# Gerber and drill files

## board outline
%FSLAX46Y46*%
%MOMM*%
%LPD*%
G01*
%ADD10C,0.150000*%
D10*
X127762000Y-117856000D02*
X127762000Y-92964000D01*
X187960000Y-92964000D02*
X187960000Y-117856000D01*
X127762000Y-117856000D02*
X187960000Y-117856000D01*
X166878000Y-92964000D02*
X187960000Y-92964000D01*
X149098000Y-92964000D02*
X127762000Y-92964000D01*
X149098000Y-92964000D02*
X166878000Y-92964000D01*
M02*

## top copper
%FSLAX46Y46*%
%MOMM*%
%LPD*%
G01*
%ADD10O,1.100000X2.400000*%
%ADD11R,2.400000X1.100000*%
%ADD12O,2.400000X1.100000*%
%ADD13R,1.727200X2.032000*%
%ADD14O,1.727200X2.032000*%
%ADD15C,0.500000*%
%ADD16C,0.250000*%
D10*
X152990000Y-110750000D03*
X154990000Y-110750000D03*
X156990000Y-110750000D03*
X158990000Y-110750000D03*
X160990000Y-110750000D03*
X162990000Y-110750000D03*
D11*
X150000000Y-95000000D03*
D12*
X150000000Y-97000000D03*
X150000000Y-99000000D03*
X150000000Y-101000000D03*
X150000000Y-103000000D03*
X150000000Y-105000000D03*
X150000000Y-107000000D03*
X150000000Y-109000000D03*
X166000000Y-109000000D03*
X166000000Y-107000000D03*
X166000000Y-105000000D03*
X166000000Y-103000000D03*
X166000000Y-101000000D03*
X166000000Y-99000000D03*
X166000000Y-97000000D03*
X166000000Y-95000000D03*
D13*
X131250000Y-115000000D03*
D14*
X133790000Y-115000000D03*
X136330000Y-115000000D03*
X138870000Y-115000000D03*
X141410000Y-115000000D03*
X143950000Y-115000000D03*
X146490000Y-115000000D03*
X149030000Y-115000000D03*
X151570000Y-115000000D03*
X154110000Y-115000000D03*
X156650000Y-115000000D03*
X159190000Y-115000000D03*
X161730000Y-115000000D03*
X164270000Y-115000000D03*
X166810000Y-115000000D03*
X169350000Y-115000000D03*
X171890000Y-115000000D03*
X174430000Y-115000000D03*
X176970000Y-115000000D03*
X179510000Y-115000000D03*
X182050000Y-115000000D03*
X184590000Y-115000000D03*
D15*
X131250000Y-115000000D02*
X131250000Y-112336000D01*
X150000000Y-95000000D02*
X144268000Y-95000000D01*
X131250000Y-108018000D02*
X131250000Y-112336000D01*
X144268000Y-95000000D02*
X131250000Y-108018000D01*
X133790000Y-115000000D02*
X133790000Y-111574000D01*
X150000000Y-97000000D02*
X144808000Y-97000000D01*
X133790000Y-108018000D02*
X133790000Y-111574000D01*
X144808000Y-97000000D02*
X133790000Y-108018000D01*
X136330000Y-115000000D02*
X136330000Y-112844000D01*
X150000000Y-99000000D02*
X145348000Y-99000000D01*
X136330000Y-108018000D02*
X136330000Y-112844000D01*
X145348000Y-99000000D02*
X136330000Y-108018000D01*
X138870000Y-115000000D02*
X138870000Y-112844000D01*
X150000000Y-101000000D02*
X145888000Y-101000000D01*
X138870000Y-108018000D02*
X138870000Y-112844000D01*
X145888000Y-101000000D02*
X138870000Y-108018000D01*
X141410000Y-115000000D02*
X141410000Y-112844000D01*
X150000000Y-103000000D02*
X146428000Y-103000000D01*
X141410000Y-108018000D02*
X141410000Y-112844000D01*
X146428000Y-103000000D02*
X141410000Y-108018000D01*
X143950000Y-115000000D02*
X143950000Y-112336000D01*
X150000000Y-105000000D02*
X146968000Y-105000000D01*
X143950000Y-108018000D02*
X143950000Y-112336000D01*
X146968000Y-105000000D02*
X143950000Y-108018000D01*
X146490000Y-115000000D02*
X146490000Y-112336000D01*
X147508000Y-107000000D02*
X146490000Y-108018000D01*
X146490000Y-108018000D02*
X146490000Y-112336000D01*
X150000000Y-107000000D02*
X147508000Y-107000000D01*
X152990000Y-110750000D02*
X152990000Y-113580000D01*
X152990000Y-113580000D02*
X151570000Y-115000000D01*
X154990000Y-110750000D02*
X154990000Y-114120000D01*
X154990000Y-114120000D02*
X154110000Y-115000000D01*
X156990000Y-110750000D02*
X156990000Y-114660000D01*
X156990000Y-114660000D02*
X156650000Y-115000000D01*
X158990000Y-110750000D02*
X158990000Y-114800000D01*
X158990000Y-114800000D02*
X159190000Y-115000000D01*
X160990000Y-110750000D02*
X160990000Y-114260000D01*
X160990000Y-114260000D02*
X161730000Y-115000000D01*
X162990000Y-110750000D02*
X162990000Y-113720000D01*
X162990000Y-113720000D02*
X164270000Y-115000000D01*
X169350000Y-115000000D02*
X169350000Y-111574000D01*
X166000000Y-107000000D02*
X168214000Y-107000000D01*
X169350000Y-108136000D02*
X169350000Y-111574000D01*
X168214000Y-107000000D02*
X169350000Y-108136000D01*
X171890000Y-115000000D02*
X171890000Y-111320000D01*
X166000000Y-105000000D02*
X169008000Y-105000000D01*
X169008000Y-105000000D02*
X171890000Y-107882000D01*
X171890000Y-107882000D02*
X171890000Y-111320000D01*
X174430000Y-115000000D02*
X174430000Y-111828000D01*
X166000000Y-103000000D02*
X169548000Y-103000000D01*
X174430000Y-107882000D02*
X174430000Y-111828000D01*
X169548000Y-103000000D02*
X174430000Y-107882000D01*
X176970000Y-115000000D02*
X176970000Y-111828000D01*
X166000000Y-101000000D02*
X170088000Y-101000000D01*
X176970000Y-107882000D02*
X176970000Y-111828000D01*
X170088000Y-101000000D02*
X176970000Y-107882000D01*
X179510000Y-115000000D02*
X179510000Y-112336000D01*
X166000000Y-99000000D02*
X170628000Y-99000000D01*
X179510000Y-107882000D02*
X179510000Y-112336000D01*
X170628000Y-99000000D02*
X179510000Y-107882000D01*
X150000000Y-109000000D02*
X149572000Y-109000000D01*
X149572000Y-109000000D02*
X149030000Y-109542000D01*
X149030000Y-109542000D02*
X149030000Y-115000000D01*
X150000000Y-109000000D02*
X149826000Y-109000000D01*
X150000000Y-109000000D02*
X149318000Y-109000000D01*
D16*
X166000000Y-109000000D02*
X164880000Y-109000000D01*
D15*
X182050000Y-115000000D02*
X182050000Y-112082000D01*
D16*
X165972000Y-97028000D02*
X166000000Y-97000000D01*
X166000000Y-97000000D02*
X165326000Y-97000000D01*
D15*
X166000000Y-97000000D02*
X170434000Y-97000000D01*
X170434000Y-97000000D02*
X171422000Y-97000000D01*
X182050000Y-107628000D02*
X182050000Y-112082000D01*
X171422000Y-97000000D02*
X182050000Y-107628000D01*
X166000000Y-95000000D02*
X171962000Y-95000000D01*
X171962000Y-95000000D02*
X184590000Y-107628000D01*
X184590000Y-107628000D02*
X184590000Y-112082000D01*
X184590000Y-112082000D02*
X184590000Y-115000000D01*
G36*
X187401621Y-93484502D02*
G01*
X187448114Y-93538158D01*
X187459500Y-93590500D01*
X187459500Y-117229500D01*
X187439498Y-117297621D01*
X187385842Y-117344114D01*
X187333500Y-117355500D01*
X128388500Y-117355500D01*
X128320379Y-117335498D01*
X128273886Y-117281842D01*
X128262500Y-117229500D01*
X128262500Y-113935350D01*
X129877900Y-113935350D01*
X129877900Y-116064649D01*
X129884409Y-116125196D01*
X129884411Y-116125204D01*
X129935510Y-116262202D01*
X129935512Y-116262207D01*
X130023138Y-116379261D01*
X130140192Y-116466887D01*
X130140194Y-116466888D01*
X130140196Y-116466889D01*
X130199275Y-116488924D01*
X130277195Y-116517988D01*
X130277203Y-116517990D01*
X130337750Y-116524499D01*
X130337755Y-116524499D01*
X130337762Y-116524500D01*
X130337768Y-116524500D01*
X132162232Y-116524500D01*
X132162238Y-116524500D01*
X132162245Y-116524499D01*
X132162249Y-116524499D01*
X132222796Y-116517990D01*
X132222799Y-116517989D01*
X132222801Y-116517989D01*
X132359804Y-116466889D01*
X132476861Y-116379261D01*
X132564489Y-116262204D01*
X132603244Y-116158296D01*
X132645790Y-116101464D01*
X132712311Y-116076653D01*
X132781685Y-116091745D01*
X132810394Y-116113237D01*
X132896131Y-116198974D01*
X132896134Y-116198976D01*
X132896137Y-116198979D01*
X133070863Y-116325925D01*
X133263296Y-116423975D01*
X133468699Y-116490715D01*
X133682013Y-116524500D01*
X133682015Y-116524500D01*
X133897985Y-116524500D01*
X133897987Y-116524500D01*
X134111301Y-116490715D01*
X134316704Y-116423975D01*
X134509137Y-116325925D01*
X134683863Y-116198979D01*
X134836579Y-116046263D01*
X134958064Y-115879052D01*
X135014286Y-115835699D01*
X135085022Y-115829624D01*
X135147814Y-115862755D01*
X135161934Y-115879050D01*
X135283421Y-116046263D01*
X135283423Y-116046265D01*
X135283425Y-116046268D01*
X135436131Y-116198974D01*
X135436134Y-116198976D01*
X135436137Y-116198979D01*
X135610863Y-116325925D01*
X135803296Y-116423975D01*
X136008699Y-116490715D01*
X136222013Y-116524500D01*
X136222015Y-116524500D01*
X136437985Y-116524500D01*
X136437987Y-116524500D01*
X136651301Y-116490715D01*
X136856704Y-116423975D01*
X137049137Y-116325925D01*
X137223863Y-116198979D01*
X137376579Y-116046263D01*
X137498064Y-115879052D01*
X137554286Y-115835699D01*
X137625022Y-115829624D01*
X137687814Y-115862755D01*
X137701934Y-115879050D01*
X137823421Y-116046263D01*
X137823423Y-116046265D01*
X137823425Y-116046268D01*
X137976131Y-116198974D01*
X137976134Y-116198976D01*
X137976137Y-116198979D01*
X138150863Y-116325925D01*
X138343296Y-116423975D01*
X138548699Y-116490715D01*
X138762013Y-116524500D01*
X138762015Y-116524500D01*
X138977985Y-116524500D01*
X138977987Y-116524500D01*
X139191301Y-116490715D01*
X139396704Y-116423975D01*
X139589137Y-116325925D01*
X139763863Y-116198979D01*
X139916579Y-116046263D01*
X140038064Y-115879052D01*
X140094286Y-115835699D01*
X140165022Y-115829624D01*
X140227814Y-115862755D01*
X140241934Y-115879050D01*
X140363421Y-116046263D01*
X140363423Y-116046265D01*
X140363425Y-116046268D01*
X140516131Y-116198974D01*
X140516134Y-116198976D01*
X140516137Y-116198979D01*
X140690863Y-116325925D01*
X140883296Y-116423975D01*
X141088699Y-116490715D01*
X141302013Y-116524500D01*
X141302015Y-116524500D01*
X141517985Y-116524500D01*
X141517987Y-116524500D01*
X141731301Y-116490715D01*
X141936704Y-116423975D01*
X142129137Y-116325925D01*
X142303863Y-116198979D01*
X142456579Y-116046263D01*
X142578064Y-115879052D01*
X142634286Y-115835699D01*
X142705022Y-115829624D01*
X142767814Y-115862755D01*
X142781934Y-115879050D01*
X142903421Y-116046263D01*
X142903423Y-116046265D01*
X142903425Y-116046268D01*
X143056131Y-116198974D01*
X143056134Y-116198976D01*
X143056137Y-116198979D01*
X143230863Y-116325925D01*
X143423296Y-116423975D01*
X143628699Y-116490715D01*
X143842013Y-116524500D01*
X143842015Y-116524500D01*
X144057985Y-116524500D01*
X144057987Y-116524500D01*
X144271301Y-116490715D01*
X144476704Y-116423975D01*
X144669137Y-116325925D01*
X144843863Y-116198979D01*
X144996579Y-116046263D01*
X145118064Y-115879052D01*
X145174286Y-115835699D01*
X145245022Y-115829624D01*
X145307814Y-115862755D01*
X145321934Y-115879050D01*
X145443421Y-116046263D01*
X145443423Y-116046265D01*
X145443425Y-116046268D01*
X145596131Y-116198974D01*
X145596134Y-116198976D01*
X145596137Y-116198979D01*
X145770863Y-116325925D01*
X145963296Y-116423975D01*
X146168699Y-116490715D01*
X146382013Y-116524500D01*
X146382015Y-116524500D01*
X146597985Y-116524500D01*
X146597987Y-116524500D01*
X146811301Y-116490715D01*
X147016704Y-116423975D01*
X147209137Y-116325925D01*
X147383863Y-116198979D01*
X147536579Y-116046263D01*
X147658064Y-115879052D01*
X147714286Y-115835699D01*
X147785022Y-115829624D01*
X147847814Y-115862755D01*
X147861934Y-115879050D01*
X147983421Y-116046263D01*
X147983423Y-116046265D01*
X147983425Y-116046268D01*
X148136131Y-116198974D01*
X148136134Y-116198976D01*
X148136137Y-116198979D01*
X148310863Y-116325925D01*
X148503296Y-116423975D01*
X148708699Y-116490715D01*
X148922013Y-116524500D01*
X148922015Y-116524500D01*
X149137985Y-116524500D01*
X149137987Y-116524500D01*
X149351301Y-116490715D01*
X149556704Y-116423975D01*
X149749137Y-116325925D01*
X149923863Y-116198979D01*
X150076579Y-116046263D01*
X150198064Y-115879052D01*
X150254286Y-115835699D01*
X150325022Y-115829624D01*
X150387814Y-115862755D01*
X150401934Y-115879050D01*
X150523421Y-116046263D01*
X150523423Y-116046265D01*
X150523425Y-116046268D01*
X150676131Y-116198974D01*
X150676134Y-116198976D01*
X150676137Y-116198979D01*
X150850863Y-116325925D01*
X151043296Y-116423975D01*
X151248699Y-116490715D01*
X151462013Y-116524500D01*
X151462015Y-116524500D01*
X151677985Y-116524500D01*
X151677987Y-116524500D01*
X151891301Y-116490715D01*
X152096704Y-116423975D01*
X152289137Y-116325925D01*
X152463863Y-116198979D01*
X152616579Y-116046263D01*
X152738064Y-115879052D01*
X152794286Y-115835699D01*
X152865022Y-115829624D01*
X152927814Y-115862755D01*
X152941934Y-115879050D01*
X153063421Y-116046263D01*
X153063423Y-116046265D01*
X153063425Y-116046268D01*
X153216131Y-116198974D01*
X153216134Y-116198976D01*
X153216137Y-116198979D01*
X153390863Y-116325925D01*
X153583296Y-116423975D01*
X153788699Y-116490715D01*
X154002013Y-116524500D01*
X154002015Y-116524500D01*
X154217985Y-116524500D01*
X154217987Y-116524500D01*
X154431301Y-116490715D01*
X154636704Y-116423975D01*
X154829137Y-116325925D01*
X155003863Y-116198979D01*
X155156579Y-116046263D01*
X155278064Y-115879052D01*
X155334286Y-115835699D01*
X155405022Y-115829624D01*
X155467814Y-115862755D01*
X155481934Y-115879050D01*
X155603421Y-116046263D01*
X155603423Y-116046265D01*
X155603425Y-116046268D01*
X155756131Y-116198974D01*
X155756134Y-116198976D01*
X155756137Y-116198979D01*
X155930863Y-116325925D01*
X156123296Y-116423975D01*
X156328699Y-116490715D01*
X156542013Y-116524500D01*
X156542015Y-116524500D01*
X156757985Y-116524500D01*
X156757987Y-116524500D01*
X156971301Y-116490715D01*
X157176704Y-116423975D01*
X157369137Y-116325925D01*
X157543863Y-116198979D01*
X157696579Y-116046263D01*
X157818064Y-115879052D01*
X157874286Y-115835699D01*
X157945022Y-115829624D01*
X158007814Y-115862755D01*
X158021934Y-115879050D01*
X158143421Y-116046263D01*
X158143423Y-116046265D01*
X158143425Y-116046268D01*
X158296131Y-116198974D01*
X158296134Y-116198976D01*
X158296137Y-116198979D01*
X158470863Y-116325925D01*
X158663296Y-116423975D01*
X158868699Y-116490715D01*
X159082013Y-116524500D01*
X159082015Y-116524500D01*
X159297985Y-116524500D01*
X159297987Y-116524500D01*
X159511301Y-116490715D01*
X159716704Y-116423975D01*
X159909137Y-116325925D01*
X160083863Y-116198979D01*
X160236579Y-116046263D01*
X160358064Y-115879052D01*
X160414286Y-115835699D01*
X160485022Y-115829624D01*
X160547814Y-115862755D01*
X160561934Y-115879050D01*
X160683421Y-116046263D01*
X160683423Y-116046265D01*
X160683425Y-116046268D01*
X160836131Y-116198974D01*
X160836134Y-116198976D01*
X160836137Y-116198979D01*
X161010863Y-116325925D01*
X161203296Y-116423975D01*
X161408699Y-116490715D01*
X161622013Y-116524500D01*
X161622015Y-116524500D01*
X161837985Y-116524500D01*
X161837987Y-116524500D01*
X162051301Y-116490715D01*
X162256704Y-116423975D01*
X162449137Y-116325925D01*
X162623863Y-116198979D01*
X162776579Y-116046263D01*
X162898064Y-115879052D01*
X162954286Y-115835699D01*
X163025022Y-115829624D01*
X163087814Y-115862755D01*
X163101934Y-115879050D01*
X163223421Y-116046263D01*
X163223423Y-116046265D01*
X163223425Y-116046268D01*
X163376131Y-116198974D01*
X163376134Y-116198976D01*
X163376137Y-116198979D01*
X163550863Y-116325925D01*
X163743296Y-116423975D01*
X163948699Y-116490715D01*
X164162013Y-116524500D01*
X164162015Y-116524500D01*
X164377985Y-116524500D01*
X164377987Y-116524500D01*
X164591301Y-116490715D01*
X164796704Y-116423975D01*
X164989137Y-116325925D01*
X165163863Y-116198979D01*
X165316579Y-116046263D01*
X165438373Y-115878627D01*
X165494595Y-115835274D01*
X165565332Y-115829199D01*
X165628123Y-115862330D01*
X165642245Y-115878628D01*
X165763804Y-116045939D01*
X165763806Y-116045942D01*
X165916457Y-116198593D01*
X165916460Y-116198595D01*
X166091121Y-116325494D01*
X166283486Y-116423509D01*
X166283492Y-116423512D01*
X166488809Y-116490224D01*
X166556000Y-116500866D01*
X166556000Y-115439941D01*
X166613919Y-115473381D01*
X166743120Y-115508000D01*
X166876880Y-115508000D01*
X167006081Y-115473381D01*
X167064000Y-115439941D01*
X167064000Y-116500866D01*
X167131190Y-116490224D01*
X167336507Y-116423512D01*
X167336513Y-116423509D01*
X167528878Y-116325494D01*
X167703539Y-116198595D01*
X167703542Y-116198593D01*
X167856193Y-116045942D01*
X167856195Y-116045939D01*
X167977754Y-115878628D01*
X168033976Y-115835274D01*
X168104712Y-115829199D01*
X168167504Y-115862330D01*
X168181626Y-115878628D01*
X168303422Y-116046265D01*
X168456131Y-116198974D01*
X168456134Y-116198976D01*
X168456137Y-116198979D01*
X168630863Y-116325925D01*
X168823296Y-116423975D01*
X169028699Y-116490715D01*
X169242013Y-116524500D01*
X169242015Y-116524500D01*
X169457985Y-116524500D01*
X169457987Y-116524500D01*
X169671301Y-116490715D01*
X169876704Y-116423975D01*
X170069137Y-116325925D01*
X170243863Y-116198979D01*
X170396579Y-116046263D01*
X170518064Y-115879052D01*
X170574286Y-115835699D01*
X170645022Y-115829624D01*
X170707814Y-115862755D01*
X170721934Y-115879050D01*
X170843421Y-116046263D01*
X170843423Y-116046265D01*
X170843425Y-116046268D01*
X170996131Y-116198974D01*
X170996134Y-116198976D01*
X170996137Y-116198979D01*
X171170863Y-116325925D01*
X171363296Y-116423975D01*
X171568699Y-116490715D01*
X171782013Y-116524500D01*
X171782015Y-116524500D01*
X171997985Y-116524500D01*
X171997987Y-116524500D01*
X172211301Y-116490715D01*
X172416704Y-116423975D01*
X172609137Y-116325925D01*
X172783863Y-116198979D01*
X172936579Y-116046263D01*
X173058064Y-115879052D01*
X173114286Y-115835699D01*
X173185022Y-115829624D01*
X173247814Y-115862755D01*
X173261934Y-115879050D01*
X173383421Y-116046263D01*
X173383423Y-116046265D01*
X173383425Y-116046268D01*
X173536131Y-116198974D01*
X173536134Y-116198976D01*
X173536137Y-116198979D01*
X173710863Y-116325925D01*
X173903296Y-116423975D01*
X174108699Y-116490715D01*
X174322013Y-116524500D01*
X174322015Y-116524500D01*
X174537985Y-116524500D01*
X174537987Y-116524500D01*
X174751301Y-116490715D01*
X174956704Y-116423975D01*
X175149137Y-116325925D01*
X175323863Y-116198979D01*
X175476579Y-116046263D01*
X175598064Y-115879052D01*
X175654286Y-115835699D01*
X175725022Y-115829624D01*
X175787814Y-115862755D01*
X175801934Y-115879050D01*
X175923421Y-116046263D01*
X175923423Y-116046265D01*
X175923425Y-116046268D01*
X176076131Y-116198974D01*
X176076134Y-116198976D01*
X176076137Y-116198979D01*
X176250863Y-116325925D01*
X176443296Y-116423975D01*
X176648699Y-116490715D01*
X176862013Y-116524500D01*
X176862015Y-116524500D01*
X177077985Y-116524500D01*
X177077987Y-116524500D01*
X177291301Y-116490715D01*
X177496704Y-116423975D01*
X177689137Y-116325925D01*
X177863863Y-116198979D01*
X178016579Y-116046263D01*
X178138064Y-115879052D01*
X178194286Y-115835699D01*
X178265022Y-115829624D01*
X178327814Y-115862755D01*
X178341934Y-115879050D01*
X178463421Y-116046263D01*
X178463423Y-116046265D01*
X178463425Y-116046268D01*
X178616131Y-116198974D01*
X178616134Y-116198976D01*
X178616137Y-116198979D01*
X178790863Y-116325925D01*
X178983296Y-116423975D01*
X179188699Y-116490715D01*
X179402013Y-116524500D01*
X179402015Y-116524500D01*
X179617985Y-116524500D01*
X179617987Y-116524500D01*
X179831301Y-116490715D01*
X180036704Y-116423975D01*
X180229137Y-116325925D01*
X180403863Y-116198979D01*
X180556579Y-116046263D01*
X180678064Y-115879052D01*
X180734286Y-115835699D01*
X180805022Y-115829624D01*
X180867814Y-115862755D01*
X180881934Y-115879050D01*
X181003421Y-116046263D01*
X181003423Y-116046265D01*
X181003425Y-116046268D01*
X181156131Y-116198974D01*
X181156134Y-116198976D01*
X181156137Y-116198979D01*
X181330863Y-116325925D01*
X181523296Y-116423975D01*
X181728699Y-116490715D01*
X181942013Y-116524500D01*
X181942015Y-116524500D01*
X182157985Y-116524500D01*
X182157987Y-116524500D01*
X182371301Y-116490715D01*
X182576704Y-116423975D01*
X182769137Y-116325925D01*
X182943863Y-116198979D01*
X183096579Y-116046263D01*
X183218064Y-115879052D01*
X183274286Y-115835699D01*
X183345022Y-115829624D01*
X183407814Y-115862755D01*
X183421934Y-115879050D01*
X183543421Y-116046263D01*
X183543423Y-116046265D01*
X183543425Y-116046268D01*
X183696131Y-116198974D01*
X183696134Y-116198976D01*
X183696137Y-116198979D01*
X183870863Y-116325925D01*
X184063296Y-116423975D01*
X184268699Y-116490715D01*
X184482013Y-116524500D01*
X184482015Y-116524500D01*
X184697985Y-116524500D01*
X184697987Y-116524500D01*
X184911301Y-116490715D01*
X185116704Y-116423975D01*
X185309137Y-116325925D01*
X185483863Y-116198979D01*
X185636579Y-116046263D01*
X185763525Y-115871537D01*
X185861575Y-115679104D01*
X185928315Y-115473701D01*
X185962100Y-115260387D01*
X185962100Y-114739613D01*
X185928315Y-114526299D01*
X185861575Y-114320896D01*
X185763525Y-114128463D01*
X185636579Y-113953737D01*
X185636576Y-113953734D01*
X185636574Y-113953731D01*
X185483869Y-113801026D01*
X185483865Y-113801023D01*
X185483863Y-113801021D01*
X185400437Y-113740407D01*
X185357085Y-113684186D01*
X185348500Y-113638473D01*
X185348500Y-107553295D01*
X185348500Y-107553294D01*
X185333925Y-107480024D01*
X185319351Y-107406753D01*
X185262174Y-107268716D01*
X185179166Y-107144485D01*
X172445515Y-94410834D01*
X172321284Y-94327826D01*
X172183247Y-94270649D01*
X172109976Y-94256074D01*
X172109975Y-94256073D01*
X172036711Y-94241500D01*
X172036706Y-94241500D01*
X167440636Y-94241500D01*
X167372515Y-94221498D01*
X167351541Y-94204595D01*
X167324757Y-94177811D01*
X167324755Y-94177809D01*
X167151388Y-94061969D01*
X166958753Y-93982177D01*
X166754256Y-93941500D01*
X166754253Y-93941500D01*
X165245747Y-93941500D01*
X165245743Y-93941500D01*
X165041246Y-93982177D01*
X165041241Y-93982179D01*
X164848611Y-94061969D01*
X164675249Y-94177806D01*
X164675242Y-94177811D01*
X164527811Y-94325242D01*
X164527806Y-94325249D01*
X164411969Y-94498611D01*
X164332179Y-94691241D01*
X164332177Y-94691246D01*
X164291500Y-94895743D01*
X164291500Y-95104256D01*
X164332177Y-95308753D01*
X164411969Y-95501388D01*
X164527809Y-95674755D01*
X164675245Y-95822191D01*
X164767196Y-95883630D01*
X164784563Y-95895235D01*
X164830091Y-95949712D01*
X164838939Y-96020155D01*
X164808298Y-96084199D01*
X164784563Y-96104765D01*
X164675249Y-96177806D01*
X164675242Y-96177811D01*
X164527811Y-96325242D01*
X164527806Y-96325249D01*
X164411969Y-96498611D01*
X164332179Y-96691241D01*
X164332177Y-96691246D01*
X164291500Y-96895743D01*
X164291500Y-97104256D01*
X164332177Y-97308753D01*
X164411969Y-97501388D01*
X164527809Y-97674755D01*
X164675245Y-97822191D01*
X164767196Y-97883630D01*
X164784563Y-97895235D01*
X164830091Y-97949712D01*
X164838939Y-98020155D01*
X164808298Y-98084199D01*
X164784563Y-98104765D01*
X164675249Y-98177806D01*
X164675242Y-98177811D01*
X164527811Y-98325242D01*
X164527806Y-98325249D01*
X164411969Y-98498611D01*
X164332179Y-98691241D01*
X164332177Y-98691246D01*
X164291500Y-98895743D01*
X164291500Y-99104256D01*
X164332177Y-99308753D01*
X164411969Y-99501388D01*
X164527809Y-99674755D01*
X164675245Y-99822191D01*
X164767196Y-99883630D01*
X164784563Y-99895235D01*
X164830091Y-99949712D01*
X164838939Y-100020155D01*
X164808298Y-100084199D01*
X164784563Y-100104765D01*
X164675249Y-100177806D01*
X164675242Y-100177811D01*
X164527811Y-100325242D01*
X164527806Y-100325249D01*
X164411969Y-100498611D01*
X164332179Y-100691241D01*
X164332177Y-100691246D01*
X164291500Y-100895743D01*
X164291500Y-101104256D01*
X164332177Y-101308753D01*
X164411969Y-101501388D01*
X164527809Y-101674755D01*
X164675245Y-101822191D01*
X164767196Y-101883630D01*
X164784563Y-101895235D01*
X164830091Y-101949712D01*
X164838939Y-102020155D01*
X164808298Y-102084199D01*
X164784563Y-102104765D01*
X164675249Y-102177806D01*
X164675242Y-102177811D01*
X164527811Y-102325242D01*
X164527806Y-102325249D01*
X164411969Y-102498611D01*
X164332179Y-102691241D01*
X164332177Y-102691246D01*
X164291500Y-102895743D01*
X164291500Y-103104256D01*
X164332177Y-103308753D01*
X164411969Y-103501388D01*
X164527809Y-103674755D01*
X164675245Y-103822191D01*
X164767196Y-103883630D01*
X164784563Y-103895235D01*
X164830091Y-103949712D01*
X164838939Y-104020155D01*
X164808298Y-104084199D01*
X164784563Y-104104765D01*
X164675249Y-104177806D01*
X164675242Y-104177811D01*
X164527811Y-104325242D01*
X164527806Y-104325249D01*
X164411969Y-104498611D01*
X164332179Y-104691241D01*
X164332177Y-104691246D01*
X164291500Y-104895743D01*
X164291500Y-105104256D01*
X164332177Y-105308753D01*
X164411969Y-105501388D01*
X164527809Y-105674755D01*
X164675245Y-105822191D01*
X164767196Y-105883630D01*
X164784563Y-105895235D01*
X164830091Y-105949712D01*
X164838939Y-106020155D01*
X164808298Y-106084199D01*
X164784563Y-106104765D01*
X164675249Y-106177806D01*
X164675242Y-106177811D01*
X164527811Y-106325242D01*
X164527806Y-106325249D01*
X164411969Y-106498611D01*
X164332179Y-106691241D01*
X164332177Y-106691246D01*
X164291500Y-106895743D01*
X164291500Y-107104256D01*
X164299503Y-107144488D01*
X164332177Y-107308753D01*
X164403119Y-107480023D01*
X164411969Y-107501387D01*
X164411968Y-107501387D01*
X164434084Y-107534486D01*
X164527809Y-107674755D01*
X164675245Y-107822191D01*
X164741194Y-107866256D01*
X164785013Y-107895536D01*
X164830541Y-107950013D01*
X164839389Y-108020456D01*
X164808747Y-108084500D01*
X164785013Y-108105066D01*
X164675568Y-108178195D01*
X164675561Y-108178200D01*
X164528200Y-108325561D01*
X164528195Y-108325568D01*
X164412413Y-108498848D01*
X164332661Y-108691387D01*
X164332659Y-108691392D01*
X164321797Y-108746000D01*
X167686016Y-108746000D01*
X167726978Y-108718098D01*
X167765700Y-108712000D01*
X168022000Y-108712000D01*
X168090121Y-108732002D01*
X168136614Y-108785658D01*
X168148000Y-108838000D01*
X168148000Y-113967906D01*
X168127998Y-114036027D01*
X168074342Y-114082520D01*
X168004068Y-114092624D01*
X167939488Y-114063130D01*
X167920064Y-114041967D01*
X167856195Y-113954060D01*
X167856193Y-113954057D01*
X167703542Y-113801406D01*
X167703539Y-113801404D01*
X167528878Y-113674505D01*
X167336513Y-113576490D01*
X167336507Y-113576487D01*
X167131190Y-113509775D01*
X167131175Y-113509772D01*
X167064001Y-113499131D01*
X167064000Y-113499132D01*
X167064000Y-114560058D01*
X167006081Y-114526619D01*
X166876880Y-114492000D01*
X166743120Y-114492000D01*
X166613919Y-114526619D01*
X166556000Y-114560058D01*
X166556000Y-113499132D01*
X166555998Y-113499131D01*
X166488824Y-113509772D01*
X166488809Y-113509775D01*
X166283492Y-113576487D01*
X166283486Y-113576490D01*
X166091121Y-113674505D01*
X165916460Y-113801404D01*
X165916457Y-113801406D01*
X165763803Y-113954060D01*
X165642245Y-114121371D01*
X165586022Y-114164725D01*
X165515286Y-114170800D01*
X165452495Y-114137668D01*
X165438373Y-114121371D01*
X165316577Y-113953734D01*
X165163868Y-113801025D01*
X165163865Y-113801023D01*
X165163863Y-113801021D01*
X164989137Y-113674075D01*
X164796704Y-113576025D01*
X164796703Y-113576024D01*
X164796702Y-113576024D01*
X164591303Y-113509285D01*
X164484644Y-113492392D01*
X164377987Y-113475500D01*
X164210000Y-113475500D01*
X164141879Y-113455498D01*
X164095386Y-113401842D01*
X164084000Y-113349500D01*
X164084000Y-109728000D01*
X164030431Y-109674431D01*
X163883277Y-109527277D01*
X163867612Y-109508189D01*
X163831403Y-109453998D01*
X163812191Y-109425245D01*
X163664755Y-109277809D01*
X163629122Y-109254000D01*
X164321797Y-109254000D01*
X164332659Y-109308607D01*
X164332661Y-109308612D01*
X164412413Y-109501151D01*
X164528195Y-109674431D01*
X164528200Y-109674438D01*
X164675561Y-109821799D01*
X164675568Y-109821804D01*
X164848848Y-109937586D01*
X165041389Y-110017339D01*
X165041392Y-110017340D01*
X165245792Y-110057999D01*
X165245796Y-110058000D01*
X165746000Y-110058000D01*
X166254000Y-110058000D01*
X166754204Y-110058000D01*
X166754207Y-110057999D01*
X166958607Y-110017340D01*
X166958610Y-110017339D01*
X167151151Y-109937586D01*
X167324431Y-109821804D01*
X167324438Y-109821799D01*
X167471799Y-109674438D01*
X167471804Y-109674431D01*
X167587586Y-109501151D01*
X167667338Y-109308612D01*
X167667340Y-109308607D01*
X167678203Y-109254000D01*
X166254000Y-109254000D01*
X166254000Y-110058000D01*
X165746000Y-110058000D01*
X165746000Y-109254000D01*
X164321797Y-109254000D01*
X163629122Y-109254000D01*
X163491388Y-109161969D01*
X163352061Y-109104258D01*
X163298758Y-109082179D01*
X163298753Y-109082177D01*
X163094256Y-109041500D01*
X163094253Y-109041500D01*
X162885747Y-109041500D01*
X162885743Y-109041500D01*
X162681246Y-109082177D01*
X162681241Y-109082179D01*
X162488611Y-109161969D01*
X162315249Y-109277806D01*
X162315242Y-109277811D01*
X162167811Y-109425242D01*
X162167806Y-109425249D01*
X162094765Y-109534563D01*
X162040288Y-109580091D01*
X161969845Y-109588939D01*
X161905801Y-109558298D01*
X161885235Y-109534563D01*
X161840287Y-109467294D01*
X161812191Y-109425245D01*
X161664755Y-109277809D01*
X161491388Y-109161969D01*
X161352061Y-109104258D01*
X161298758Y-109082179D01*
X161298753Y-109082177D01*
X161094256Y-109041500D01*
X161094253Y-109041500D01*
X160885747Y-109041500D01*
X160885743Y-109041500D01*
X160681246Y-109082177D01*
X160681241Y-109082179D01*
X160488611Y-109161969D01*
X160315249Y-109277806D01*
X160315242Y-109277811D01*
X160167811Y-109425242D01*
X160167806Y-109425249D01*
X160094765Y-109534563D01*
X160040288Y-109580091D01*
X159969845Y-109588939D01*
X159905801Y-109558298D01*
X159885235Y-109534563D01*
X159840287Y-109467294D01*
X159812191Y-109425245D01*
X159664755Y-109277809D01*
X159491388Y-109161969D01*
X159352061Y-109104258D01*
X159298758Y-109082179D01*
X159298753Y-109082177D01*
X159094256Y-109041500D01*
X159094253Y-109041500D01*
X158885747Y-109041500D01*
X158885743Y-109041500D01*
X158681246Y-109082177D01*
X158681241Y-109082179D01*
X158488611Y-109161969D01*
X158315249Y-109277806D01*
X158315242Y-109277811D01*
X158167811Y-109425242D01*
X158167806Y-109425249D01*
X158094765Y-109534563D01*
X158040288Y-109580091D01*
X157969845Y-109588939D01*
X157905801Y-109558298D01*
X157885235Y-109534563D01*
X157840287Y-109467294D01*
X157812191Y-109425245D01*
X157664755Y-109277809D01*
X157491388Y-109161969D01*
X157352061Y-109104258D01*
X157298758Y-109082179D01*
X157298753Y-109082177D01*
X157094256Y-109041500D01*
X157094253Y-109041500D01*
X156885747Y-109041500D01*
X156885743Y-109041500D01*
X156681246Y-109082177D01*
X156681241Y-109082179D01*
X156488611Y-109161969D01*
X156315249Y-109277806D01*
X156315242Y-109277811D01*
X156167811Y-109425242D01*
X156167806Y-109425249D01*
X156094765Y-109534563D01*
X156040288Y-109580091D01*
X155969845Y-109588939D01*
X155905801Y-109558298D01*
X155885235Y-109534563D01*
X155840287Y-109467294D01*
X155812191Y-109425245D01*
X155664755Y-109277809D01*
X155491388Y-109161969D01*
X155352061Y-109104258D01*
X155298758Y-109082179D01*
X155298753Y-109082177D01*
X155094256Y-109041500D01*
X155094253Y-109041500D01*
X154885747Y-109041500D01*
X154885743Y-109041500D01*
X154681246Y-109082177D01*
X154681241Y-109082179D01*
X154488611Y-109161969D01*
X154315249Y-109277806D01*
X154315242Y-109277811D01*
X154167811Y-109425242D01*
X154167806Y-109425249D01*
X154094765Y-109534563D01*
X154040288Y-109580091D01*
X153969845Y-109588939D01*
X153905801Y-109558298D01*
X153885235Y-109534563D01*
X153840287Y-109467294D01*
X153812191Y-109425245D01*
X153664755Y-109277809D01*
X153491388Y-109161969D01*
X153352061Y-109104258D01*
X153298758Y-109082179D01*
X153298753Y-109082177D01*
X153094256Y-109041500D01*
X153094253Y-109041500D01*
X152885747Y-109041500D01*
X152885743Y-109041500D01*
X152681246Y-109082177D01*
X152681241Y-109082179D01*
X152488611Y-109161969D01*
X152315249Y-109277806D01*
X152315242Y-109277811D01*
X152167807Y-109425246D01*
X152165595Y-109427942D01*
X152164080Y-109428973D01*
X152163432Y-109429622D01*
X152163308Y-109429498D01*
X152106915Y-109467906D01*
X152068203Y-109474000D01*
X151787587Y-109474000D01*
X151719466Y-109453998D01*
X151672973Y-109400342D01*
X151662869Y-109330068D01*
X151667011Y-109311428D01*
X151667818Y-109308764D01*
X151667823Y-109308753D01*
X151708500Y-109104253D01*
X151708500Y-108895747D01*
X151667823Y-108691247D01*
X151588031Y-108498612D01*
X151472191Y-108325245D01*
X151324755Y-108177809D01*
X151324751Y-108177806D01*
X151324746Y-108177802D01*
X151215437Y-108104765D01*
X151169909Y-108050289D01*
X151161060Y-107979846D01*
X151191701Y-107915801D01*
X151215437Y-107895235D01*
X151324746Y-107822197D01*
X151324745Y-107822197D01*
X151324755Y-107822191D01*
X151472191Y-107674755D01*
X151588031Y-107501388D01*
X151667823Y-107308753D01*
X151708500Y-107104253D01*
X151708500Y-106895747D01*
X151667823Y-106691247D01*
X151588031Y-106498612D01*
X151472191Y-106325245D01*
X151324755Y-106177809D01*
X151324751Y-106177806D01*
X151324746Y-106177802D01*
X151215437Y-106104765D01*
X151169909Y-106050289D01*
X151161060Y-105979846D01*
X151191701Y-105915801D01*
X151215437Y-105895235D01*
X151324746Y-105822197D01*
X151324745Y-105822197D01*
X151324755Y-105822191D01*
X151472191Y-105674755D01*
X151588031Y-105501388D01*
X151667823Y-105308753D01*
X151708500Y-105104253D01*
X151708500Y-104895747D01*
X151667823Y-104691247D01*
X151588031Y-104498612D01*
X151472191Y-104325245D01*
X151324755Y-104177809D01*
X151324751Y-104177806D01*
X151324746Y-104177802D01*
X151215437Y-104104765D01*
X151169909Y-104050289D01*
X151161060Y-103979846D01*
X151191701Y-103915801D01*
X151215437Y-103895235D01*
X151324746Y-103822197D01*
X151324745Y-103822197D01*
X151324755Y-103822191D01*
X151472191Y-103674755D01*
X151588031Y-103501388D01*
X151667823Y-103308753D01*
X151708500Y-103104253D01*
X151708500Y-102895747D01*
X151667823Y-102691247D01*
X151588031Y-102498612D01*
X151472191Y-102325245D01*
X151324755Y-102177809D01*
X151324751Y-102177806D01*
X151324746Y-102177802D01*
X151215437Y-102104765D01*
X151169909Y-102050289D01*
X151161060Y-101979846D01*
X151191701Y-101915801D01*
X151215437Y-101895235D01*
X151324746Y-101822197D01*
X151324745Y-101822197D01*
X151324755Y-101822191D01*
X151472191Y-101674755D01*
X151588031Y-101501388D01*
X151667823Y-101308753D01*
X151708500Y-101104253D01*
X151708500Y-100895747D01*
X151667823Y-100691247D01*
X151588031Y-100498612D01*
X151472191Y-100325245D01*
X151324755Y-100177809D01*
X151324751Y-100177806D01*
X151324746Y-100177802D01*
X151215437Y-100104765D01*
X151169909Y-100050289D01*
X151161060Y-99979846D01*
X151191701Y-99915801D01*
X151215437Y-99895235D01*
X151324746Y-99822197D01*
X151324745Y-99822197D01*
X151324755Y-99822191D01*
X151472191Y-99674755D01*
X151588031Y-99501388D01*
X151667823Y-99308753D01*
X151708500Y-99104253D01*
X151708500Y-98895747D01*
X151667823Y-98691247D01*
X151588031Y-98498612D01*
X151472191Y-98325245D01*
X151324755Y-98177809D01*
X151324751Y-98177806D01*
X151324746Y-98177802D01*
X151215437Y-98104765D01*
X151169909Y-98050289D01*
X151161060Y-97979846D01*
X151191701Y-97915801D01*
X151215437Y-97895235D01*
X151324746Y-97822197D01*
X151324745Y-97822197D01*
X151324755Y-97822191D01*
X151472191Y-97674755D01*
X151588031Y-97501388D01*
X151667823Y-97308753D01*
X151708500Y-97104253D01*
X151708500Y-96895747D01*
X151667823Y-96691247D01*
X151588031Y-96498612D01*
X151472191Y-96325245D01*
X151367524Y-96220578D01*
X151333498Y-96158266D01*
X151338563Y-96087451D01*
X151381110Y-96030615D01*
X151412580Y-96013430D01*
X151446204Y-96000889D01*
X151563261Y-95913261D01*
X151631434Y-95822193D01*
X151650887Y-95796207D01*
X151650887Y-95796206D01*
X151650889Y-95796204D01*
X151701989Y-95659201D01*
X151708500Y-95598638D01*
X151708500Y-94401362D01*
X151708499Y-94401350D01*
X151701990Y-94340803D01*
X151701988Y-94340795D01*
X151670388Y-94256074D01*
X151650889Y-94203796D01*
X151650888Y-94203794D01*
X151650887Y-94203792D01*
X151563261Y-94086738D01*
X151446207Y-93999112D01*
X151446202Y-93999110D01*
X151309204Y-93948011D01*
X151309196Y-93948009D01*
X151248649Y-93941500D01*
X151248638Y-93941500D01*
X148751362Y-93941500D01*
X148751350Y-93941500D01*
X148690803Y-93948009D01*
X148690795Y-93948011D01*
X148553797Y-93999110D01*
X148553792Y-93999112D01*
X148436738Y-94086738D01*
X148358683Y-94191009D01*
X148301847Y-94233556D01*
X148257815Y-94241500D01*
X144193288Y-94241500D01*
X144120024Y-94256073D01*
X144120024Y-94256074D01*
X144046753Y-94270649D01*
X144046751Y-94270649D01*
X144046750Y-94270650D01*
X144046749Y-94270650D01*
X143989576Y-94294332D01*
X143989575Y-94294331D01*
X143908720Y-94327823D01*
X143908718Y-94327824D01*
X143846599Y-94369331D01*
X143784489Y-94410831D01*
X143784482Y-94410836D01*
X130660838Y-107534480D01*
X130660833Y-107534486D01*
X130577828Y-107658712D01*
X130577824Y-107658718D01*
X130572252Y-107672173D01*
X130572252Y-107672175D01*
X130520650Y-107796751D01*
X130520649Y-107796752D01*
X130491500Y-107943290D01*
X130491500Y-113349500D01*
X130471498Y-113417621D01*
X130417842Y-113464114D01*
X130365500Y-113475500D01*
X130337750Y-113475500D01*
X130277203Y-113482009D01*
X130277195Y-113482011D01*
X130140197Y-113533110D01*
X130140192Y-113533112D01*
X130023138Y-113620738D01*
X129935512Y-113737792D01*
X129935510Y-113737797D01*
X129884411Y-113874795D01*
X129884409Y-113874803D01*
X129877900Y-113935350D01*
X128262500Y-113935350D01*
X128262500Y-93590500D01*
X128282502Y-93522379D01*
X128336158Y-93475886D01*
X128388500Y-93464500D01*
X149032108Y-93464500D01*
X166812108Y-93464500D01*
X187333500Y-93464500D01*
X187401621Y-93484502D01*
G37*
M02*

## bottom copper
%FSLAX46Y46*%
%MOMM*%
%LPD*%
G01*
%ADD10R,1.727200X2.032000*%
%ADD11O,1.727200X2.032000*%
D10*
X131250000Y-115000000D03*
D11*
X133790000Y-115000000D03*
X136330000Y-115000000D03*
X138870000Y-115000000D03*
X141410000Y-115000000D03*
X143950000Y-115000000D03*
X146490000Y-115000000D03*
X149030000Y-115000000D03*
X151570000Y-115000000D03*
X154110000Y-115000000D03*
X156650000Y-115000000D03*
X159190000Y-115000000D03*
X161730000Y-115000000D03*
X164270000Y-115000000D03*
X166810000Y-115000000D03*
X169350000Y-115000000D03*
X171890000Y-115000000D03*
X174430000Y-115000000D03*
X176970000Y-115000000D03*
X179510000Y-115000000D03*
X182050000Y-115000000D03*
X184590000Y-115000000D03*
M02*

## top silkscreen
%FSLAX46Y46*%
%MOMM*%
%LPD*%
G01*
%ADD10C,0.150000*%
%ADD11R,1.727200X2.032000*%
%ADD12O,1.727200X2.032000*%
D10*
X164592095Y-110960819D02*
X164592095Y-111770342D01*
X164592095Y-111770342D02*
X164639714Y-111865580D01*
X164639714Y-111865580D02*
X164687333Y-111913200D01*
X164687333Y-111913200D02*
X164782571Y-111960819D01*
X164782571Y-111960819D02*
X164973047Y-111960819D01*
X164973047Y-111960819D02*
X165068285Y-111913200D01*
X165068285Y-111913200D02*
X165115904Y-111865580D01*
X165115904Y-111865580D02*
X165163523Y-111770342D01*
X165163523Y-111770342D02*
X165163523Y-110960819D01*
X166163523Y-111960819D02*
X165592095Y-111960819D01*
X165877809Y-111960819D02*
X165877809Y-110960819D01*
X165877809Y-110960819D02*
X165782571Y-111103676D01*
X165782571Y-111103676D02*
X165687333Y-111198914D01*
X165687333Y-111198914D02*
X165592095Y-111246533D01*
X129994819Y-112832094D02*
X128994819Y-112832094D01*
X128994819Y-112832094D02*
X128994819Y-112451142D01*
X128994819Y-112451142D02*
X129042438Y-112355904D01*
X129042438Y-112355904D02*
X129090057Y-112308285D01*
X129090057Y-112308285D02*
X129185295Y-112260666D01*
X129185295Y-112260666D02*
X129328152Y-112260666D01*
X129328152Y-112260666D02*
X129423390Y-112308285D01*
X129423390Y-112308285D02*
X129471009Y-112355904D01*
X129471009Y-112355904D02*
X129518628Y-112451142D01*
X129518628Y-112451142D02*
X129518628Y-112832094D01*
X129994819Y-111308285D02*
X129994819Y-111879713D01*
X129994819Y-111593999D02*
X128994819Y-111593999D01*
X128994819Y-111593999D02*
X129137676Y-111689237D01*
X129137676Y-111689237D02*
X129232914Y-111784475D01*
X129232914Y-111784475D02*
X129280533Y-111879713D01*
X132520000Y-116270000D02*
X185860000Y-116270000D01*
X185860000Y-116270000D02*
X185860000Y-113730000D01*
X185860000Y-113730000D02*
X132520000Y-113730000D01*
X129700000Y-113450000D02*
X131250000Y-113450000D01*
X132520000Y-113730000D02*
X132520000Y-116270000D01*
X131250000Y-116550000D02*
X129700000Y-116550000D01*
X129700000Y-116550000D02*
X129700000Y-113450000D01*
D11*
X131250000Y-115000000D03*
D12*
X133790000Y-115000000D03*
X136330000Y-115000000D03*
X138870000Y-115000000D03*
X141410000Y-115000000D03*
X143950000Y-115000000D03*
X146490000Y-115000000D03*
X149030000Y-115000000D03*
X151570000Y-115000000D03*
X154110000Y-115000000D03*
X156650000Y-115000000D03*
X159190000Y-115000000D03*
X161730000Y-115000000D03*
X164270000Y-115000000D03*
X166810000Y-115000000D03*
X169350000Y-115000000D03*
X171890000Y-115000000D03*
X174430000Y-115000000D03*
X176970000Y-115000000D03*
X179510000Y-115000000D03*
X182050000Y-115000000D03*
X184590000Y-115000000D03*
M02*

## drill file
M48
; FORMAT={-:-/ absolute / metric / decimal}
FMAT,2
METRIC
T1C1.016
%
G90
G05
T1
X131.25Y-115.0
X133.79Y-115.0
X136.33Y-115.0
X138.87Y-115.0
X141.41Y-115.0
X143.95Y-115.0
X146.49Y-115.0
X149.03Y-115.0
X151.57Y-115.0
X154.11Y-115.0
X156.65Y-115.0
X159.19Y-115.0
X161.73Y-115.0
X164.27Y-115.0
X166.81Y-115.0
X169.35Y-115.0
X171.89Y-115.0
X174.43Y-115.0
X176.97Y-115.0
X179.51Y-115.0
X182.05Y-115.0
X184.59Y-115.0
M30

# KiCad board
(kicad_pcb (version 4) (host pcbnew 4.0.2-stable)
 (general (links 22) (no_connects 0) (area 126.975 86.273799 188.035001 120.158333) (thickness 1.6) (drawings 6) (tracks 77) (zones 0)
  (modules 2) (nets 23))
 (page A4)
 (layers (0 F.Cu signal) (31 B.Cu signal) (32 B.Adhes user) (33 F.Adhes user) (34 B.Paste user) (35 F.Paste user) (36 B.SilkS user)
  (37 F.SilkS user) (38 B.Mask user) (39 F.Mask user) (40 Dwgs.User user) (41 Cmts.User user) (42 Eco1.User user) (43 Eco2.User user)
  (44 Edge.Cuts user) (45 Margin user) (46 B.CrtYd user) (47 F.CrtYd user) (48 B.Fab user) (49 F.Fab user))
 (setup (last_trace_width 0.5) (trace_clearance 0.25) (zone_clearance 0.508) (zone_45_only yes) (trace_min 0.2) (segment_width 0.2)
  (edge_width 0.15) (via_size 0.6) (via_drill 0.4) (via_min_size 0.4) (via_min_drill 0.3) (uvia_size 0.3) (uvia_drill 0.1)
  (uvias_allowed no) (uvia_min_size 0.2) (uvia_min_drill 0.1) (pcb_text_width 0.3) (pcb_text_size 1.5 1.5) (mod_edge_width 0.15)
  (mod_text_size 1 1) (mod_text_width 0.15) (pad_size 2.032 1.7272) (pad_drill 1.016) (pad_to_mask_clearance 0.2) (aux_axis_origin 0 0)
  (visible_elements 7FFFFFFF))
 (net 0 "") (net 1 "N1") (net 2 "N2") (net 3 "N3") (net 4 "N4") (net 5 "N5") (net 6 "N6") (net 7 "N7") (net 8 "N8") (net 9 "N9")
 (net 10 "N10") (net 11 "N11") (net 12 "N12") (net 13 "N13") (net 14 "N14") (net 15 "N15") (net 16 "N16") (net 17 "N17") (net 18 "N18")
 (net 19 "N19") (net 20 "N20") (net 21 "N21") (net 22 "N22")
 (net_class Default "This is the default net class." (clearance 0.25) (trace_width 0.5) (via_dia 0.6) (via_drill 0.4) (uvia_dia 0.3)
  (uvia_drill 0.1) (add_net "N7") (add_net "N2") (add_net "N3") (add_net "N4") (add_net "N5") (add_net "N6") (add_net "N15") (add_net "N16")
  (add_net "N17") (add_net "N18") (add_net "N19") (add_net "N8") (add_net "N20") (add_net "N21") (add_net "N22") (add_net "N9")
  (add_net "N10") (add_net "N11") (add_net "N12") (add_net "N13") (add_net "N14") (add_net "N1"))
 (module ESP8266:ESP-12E (layer F.Cu) (at 150 95)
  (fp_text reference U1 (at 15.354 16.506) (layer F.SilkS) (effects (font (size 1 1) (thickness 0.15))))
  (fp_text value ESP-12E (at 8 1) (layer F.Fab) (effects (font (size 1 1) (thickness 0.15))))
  (pad 9 smd oval (at 2.99 15.75 90) (size 2.4 1.1) (layers F.Cu F.Paste F.Mask) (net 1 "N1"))
  (pad 10 smd oval (at 4.99 15.75 90) (size 2.4 1.1) (layers F.Cu F.Paste F.Mask) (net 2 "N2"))
  (pad 11 smd oval (at 6.99 15.75 90) (size 2.4 1.1) (layers F.Cu F.Paste F.Mask) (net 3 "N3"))
  (pad 12 smd oval (at 8.99 15.75 90) (size 2.4 1.1) (layers F.Cu F.Paste F.Mask) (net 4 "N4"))
  (pad 13 smd oval (at 10.99 15.75 90) (size 2.4 1.1) (layers F.Cu F.Paste F.Mask) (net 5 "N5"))
  (pad 14 smd oval (at 12.99 15.75 90) (size 2.4 1.1) (layers F.Cu F.Paste F.Mask) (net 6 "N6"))
  (pad 1 smd rect (at 0 0) (size 2.4 1.1) (layers F.Cu F.Paste F.Mask) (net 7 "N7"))
  (pad 2 smd oval (at 0 2) (size 2.4 1.1) (layers F.Cu F.Paste F.Mask) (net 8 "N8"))
  (pad 3 smd oval (at 0 4) (size 2.4 1.1) (layers F.Cu F.Paste F.Mask) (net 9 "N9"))
  (pad 4 smd oval (at 0 6) (size 2.4 1.1) (layers F.Cu F.Paste F.Mask) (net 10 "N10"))
  (pad 5 smd oval (at 0 8) (size 2.4 1.1) (layers F.Cu F.Paste F.Mask) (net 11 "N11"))
  (pad 6 smd oval (at 0 10) (size 2.4 1.1) (layers F.Cu F.Paste F.Mask) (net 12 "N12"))
  (pad 7 smd oval (at 0 12) (size 2.4 1.1) (layers F.Cu F.Paste F.Mask) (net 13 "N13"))
  (pad 8 smd oval (at 0 14) (size 2.4 1.1) (layers F.Cu F.Paste F.Mask) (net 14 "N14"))
  (pad 15 smd oval (at 16 14) (size 2.4 1.1) (layers F.Cu F.Paste F.Mask) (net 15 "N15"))
  (pad 16 smd oval (at 16 12) (size 2.4 1.1) (layers F.Cu F.Paste F.Mask) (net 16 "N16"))
  (pad 17 smd oval (at 16 10) (size 2.4 1.1) (layers F.Cu F.Paste F.Mask) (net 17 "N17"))
  (pad 18 smd oval (at 16 8) (size 2.4 1.1) (layers F.Cu F.Paste F.Mask) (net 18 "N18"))
  (pad 19 smd oval (at 16 6) (size 2.4 1.1) (layers F.Cu F.Paste F.Mask) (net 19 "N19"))
  (pad 20 smd oval (at 16 4) (size 2.4 1.1) (layers F.Cu F.Paste F.Mask) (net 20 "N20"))
  (pad 21 smd oval (at 16 2) (size 2.4 1.1) (layers F.Cu F.Paste F.Mask) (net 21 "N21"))
  (pad 22 smd oval (at 16 0) (size 2.4 1.1) (layers F.Cu F.Paste F.Mask) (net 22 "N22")))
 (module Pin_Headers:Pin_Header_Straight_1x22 (layer F.Cu) (at 131.25 115 90)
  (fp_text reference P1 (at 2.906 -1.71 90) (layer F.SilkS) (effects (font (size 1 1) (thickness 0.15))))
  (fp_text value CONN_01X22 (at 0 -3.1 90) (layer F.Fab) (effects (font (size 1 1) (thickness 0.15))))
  (fp_line (start -1.27 1.27) (end -1.27 54.61) (layer F.SilkS) (width 0.15))
  (fp_line (start -1.27 54.61) (end 1.27 54.61) (layer F.SilkS) (width 0.15))
  (fp_line (start 1.27 54.61) (end 1.27 1.27) (layer F.SilkS) (width 0.15))
  (fp_line (start 1.55 -1.55) (end 1.55 0) (layer F.SilkS) (width 0.15))
  (fp_line (start 1.27 1.27) (end -1.27 1.27) (layer F.SilkS) (width 0.15))
  (fp_line (start -1.55 0) (end -1.55 -1.55) (layer F.SilkS) (width 0.15))
  (fp_line (start -1.55 -1.55) (end 1.55 -1.55) (layer F.SilkS) (width 0.15))
  (pad 1 thru_hole rect (at 0 0 90) (size 2.032 1.7272) (drill 1.016) (layers *.Cu *.Mask F.SilkS) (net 7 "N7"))
  (pad 2 thru_hole oval (at 0 2.54 90) (size 2.032 1.7272) (drill 1.016) (layers *.Cu *.Mask F.SilkS) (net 8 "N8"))
  (pad 3 thru_hole oval (at 0 5.08 90) (size 2.032 1.7272) (drill 1.016) (layers *.Cu *.Mask F.SilkS) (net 9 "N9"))
  (pad 4 thru_hole oval (at 0 7.62 90) (size 2.032 1.7272) (drill 1.016) (layers *.Cu *.Mask F.SilkS) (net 10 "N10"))
  (pad 5 thru_hole oval (at 0 10.16 90) (size 2.032 1.7272) (drill 1.016) (layers *.Cu *.Mask F.SilkS) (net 11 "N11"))
  (pad 6 thru_hole oval (at 0 12.7 90) (size 2.032 1.7272) (drill 1.016) (layers *.Cu *.Mask F.SilkS) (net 12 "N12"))
  (pad 7 thru_hole oval (at 0 15.24 90) (size 2.032 1.7272) (drill 1.016) (layers *.Cu *.Mask F.SilkS) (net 13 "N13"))
  (pad 8 thru_hole oval (at 0 17.78 90) (size 2.032 1.7272) (drill 1.016) (layers *.Cu *.Mask F.SilkS) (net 14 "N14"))
  (pad 9 thru_hole oval (at 0 20.32 90) (size 2.032 1.7272) (drill 1.016) (layers *.Cu *.Mask F.SilkS) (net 1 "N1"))
  (pad 10 thru_hole oval (at 0 22.86 90) (size 2.032 1.7272) (drill 1.016) (layers *.Cu *.Mask F.SilkS) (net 2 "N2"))
  (pad 11 thru_hole oval (at 0 25.4 90) (size 2.032 1.7272) (drill 1.016) (layers *.Cu *.Mask F.SilkS) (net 3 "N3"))
  (pad 12 thru_hole oval (at 0 27.94 90) (size 2.032 1.7272) (drill 1.016) (layers *.Cu *.Mask F.SilkS) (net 4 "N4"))
  (pad 13 thru_hole oval (at 0 30.48 90) (size 2.032 1.7272) (drill 1.016) (layers *.Cu *.Mask F.SilkS) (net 5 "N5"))
  (pad 14 thru_hole oval (at 0 33.02 90) (size 2.032 1.7272) (drill 1.016) (layers *.Cu *.Mask F.SilkS) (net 6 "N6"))
  (pad 15 thru_hole oval (at 0 35.56 90) (size 2.032 1.7272) (drill 1.016) (layers *.Cu *.Mask F.SilkS) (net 15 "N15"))
  (pad 16 thru_hole oval (at 0 38.1 90) (size 2.032 1.7272) (drill 1.016) (layers *.Cu *.Mask F.SilkS) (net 16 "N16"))
  (pad 17 thru_hole oval (at 0 40.64 90) (size 2.032 1.7272) (drill 1.016) (layers *.Cu *.Mask F.SilkS) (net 17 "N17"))
  (pad 18 thru_hole oval (at 0 43.18 90) (size 2.032 1.7272) (drill 1.016) (layers *.Cu *.Mask F.SilkS) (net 18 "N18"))
  (pad 19 thru_hole oval (at 0 45.72 90) (size 2.032 1.7272) (drill 1.016) (layers *.Cu *.Mask F.SilkS) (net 19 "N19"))
  (pad 20 thru_hole oval (at 0 48.26 90) (size 2.032 1.7272) (drill 1.016) (layers *.Cu *.Mask F.SilkS) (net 20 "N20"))
  (pad 21 thru_hole oval (at 0 50.8 90) (size 2.032 1.7272) (drill 1.016) (layers *.Cu *.Mask F.SilkS) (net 21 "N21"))
  (pad 22 thru_hole oval (at 0 53.34 90) (size 2.032 1.7272) (drill 1.016) (layers *.Cu *.Mask F.SilkS) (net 22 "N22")))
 (gr_line (start 127.762 117.856) (end 127.762 92.964) (angle 90) (layer Edge.Cuts) (width 0.15))
 (gr_line (start 187.96 92.964) (end 187.96 117.856) (angle 90) (layer Edge.Cuts) (width 0.15))
 (gr_line (start 127.762 117.856) (end 187.96 117.856) (angle 90) (layer Edge.Cuts) (width 0.15))
 (gr_line (start 166.878 92.964) (end 187.96 92.964) (angle 90) (layer Edge.Cuts) (width 0.15))
 (gr_line (start 149.098 92.964) (end 127.762 92.964) (angle 90) (layer Edge.Cuts) (width 0.15))
 (gr_line (start 149.098 92.964) (end 166.878 92.964) (angle 90) (layer Edge.Cuts) (width 0.15))
 (segment (start 131.25 115) (end 131.25 112.336) (width 0.5) (layer F.Cu) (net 7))
 (segment (start 150 95) (end 144.268 95) (width 0.5) (layer F.Cu) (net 7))
 (segment (start 131.25 108.018) (end 131.25 112.336) (width 0.5) (layer F.Cu) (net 7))
 (segment (start 144.268 95) (end 131.25 108.018) (width 0.5) (layer F.Cu) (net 7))
 (segment (start 133.79 115) (end 133.79 111.574) (width 0.5) (layer F.Cu) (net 8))
 (segment (start 150 97) (end 144.808 97) (width 0.5) (layer F.Cu) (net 8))
 (segment (start 133.79 108.018) (end 133.79 111.574) (width 0.5) (layer F.Cu) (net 8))
 (segment (start 144.808 97) (end 133.79 108.018) (width 0.5) (layer F.Cu) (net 8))
 (segment (start 136.33 115) (end 136.33 112.844) (width 0.5) (layer F.Cu) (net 9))
 (segment (start 150 99) (end 145.348 99) (width 0.5) (layer F.Cu) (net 9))
 (segment (start 136.33 108.018) (end 136.33 112.844) (width 0.5) (layer F.Cu) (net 9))
 (segment (start 145.348 99) (end 136.33 108.018) (width 0.5) (layer F.Cu) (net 9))
 (segment (start 138.87 115) (end 138.87 112.844) (width 0.5) (layer F.Cu) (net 10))
 (segment (start 150 101) (end 145.888 101) (width 0.5) (layer F.Cu) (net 10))
 (segment (start 138.87 108.018) (end 138.87 112.844) (width 0.5) (layer F.Cu) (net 10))
 (segment (start 145.888 101) (end 138.87 108.018) (width 0.5) (layer F.Cu) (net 10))
 (segment (start 141.41 115) (end 141.41 112.844) (width 0.5) (layer F.Cu) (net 11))
 (segment (start 150 103) (end 146.428 103) (width 0.5) (layer F.Cu) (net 11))
 (segment (start 141.41 108.018) (end 141.41 112.844) (width 0.5) (layer F.Cu) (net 11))
 (segment (start 146.428 103) (end 141.41 108.018) (width 0.5) (layer F.Cu) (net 11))
 (segment (start 143.95 115) (end 143.95 112.336) (width 0.5) (layer F.Cu) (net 12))
 (segment (start 150 105) (end 146.968 105) (width 0.5) (layer F.Cu) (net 12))
 (segment (start 143.95 108.018) (end 143.95 112.336) (width 0.5) (layer F.Cu) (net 12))
 (segment (start 146.968 105) (end 143.95 108.018) (width 0.5) (layer F.Cu) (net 12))
 (segment (start 146.49 115) (end 146.49 112.336) (width 0.5) (layer F.Cu) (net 13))
 (segment (start 147.508 107) (end 146.49 108.018) (width 0.5) (layer F.Cu) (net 13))
 (segment (start 146.49 108.018) (end 146.49 112.336) (width 0.5) (layer F.Cu) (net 13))
 (segment (start 150 107) (end 147.508 107) (width 0.5) (layer F.Cu) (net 13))
 (segment (start 152.99 110.75) (end 152.99 113.58) (width 0.5) (layer F.Cu) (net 1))
 (segment (start 152.99 113.58) (end 151.57 115) (width 0.5) (layer F.Cu) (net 1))
 (segment (start 154.99 110.75) (end 154.99 114.12) (width 0.5) (layer F.Cu) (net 2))
 (segment (start 154.99 114.12) (end 154.11 115) (width 0.5) (layer F.Cu) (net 2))
 (segment (start 156.99 110.75) (end 156.99 114.66) (width 0.5) (layer F.Cu) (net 3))
 (segment (start 156.99 114.66) (end 156.65 115) (width 0.5) (layer F.Cu) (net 3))
 (segment (start 158.99 110.75) (end 158.99 114.8) (width 0.5) (layer F.Cu) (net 4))
 (segment (start 158.99 114.8) (end 159.19 115) (width 0.5) (layer F.Cu) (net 4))
 (segment (start 160.99 110.75) (end 160.99 114.26) (width 0.5) (layer F.Cu) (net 5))
 (segment (start 160.99 114.26) (end 161.73 115) (width 0.5) (layer F.Cu) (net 5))
 (segment (start 162.99 110.75) (end 162.99 113.72) (width 0.5) (layer F.Cu) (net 6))
 (segment (start 162.99 113.72) (end 164.27 115) (width 0.5) (layer F.Cu) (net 6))
 (segment (start 169.35 115) (end 169.35 111.574) (width 0.5) (layer F.Cu) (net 16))
 (segment (start 166 107) (end 168.214 107) (width 0.5) (layer F.Cu) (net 16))
 (segment (start 169.35 108.136) (end 169.35 111.574) (width 0.5) (layer F.Cu) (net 16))
 (segment (start 168.214 107) (end 169.35 108.136) (width 0.5) (layer F.Cu) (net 16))
 (segment (start 171.89 115) (end 171.89 111.32) (width 0.5) (layer F.Cu) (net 17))
 (segment (start 166 105) (end 169.008 105) (width 0.5) (layer F.Cu) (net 17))
 (segment (start 169.008 105) (end 171.89 107.882) (width 0.5) (layer F.Cu) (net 17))
 (segment (start 171.89 107.882) (end 171.89 111.32) (width 0.5) (layer F.Cu) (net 17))
 (segment (start 174.43 115) (end 174.43 111.828) (width 0.5) (layer F.Cu) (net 18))
 (segment (start 166 103) (end 169.548 103) (width 0.5) (layer F.Cu) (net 18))
 (segment (start 174.43 107.882) (end 174.43 111.828) (width 0.5) (layer F.Cu) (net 18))
 (segment (start 169.548 103) (end 174.43 107.882) (width 0.5) (layer F.Cu) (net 18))
 (segment (start 176.97 115) (end 176.97 111.828) (width 0.5) (layer F.Cu) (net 19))
 (segment (start 166 101) (end 170.088 101) (width 0.5) (layer F.Cu) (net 19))
 (segment (start 176.97 107.882) (end 176.97 111.828) (width 0.5) (layer F.Cu) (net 19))
 (segment (start 170.088 101) (end 176.97 107.882) (width 0.5) (layer F.Cu) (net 19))
 (segment (start 179.51 115) (end 179.51 112.336) (width 0.5) (layer F.Cu) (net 20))
 (segment (start 166 99) (end 170.628 99) (width 0.5) (layer F.Cu) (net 20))
 (segment (start 179.51 107.882) (end 179.51 112.336) (width 0.5) (layer F.Cu) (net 20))
 (segment (start 170.628 99) (end 179.51 107.882) (width 0.5) (layer F.Cu) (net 20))
 (segment (start 150 109) (end 149.572 109) (width 0.5) (layer F.Cu) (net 14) (status C00000))
 (segment (start 149.572 109) (end 149.03 109.542) (width 0.5) (layer F.Cu) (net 14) (status 400000))
 (segment (start 149.03 109.542) (end 149.03 115) (width 0.5) (layer F.Cu) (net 14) (status 800000))
 (segment (start 150 109) (end 149.826 109) (width 0.5) (layer F.Cu) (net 14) (status C00000))
 (segment (start 150 109) (end 149.318 109) (width 0.5) (layer F.Cu) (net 14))
 (segment (start 166 109) (end 164.88 109) (width 0.25) (layer F.Cu) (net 15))
 (segment (start 182.05 115) (end 182.05 112.082) (width 0.5) (layer F.Cu) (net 21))
 (segment (start 165.972 97.028) (end 166 97) (width 0.25) (layer F.Cu) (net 21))
 (segment (start 166 97) (end 165.326 97) (width 0.25) (layer F.Cu) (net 21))
 (segment (start 166 97) (end 170.434 97) (width 0.5) (layer F.Cu) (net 21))
 (segment (start 170.434 97) (end 171.422 97) (width 0.5) (layer F.Cu) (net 21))
 (segment (start 182.05 107.628) (end 182.05 112.082) (width 0.5) (layer F.Cu) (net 21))
 (segment (start 171.422 97) (end 182.05 107.628) (width 0.5) (layer F.Cu) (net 21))
 (segment (start 166 95) (end 171.962 95) (width 0.5) (layer F.Cu) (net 22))
 (segment (start 171.962 95) (end 184.59 107.628) (width 0.5) (layer F.Cu) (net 22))
 (segment (start 184.59 107.628) (end 184.59 112.082) (width 0.5) (layer F.Cu) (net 22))
 (segment (start 184.59 112.082) (end 184.59 115) (width 0.5) (layer F.Cu) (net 22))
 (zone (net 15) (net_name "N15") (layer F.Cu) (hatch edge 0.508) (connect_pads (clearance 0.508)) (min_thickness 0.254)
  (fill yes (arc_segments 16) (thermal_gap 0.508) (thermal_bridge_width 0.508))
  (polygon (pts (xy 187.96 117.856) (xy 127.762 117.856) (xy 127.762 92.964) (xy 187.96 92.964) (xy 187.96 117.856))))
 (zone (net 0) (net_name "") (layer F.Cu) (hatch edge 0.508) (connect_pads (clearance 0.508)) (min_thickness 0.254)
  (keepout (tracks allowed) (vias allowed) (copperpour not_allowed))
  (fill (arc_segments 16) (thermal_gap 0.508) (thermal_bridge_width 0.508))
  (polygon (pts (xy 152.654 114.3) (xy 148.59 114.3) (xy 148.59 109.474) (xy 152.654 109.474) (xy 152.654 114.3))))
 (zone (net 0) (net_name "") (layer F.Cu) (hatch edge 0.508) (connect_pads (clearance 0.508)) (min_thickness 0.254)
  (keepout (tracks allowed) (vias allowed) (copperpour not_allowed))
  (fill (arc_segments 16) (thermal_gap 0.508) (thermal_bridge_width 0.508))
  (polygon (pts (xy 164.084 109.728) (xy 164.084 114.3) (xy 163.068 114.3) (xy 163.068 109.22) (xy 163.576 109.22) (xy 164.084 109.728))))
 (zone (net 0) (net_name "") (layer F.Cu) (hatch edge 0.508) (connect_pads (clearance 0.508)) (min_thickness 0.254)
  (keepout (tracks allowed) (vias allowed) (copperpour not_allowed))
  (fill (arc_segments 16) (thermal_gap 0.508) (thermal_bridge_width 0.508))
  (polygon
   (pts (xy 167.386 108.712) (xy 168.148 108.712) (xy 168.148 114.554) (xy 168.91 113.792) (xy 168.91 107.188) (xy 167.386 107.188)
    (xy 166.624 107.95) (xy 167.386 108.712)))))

